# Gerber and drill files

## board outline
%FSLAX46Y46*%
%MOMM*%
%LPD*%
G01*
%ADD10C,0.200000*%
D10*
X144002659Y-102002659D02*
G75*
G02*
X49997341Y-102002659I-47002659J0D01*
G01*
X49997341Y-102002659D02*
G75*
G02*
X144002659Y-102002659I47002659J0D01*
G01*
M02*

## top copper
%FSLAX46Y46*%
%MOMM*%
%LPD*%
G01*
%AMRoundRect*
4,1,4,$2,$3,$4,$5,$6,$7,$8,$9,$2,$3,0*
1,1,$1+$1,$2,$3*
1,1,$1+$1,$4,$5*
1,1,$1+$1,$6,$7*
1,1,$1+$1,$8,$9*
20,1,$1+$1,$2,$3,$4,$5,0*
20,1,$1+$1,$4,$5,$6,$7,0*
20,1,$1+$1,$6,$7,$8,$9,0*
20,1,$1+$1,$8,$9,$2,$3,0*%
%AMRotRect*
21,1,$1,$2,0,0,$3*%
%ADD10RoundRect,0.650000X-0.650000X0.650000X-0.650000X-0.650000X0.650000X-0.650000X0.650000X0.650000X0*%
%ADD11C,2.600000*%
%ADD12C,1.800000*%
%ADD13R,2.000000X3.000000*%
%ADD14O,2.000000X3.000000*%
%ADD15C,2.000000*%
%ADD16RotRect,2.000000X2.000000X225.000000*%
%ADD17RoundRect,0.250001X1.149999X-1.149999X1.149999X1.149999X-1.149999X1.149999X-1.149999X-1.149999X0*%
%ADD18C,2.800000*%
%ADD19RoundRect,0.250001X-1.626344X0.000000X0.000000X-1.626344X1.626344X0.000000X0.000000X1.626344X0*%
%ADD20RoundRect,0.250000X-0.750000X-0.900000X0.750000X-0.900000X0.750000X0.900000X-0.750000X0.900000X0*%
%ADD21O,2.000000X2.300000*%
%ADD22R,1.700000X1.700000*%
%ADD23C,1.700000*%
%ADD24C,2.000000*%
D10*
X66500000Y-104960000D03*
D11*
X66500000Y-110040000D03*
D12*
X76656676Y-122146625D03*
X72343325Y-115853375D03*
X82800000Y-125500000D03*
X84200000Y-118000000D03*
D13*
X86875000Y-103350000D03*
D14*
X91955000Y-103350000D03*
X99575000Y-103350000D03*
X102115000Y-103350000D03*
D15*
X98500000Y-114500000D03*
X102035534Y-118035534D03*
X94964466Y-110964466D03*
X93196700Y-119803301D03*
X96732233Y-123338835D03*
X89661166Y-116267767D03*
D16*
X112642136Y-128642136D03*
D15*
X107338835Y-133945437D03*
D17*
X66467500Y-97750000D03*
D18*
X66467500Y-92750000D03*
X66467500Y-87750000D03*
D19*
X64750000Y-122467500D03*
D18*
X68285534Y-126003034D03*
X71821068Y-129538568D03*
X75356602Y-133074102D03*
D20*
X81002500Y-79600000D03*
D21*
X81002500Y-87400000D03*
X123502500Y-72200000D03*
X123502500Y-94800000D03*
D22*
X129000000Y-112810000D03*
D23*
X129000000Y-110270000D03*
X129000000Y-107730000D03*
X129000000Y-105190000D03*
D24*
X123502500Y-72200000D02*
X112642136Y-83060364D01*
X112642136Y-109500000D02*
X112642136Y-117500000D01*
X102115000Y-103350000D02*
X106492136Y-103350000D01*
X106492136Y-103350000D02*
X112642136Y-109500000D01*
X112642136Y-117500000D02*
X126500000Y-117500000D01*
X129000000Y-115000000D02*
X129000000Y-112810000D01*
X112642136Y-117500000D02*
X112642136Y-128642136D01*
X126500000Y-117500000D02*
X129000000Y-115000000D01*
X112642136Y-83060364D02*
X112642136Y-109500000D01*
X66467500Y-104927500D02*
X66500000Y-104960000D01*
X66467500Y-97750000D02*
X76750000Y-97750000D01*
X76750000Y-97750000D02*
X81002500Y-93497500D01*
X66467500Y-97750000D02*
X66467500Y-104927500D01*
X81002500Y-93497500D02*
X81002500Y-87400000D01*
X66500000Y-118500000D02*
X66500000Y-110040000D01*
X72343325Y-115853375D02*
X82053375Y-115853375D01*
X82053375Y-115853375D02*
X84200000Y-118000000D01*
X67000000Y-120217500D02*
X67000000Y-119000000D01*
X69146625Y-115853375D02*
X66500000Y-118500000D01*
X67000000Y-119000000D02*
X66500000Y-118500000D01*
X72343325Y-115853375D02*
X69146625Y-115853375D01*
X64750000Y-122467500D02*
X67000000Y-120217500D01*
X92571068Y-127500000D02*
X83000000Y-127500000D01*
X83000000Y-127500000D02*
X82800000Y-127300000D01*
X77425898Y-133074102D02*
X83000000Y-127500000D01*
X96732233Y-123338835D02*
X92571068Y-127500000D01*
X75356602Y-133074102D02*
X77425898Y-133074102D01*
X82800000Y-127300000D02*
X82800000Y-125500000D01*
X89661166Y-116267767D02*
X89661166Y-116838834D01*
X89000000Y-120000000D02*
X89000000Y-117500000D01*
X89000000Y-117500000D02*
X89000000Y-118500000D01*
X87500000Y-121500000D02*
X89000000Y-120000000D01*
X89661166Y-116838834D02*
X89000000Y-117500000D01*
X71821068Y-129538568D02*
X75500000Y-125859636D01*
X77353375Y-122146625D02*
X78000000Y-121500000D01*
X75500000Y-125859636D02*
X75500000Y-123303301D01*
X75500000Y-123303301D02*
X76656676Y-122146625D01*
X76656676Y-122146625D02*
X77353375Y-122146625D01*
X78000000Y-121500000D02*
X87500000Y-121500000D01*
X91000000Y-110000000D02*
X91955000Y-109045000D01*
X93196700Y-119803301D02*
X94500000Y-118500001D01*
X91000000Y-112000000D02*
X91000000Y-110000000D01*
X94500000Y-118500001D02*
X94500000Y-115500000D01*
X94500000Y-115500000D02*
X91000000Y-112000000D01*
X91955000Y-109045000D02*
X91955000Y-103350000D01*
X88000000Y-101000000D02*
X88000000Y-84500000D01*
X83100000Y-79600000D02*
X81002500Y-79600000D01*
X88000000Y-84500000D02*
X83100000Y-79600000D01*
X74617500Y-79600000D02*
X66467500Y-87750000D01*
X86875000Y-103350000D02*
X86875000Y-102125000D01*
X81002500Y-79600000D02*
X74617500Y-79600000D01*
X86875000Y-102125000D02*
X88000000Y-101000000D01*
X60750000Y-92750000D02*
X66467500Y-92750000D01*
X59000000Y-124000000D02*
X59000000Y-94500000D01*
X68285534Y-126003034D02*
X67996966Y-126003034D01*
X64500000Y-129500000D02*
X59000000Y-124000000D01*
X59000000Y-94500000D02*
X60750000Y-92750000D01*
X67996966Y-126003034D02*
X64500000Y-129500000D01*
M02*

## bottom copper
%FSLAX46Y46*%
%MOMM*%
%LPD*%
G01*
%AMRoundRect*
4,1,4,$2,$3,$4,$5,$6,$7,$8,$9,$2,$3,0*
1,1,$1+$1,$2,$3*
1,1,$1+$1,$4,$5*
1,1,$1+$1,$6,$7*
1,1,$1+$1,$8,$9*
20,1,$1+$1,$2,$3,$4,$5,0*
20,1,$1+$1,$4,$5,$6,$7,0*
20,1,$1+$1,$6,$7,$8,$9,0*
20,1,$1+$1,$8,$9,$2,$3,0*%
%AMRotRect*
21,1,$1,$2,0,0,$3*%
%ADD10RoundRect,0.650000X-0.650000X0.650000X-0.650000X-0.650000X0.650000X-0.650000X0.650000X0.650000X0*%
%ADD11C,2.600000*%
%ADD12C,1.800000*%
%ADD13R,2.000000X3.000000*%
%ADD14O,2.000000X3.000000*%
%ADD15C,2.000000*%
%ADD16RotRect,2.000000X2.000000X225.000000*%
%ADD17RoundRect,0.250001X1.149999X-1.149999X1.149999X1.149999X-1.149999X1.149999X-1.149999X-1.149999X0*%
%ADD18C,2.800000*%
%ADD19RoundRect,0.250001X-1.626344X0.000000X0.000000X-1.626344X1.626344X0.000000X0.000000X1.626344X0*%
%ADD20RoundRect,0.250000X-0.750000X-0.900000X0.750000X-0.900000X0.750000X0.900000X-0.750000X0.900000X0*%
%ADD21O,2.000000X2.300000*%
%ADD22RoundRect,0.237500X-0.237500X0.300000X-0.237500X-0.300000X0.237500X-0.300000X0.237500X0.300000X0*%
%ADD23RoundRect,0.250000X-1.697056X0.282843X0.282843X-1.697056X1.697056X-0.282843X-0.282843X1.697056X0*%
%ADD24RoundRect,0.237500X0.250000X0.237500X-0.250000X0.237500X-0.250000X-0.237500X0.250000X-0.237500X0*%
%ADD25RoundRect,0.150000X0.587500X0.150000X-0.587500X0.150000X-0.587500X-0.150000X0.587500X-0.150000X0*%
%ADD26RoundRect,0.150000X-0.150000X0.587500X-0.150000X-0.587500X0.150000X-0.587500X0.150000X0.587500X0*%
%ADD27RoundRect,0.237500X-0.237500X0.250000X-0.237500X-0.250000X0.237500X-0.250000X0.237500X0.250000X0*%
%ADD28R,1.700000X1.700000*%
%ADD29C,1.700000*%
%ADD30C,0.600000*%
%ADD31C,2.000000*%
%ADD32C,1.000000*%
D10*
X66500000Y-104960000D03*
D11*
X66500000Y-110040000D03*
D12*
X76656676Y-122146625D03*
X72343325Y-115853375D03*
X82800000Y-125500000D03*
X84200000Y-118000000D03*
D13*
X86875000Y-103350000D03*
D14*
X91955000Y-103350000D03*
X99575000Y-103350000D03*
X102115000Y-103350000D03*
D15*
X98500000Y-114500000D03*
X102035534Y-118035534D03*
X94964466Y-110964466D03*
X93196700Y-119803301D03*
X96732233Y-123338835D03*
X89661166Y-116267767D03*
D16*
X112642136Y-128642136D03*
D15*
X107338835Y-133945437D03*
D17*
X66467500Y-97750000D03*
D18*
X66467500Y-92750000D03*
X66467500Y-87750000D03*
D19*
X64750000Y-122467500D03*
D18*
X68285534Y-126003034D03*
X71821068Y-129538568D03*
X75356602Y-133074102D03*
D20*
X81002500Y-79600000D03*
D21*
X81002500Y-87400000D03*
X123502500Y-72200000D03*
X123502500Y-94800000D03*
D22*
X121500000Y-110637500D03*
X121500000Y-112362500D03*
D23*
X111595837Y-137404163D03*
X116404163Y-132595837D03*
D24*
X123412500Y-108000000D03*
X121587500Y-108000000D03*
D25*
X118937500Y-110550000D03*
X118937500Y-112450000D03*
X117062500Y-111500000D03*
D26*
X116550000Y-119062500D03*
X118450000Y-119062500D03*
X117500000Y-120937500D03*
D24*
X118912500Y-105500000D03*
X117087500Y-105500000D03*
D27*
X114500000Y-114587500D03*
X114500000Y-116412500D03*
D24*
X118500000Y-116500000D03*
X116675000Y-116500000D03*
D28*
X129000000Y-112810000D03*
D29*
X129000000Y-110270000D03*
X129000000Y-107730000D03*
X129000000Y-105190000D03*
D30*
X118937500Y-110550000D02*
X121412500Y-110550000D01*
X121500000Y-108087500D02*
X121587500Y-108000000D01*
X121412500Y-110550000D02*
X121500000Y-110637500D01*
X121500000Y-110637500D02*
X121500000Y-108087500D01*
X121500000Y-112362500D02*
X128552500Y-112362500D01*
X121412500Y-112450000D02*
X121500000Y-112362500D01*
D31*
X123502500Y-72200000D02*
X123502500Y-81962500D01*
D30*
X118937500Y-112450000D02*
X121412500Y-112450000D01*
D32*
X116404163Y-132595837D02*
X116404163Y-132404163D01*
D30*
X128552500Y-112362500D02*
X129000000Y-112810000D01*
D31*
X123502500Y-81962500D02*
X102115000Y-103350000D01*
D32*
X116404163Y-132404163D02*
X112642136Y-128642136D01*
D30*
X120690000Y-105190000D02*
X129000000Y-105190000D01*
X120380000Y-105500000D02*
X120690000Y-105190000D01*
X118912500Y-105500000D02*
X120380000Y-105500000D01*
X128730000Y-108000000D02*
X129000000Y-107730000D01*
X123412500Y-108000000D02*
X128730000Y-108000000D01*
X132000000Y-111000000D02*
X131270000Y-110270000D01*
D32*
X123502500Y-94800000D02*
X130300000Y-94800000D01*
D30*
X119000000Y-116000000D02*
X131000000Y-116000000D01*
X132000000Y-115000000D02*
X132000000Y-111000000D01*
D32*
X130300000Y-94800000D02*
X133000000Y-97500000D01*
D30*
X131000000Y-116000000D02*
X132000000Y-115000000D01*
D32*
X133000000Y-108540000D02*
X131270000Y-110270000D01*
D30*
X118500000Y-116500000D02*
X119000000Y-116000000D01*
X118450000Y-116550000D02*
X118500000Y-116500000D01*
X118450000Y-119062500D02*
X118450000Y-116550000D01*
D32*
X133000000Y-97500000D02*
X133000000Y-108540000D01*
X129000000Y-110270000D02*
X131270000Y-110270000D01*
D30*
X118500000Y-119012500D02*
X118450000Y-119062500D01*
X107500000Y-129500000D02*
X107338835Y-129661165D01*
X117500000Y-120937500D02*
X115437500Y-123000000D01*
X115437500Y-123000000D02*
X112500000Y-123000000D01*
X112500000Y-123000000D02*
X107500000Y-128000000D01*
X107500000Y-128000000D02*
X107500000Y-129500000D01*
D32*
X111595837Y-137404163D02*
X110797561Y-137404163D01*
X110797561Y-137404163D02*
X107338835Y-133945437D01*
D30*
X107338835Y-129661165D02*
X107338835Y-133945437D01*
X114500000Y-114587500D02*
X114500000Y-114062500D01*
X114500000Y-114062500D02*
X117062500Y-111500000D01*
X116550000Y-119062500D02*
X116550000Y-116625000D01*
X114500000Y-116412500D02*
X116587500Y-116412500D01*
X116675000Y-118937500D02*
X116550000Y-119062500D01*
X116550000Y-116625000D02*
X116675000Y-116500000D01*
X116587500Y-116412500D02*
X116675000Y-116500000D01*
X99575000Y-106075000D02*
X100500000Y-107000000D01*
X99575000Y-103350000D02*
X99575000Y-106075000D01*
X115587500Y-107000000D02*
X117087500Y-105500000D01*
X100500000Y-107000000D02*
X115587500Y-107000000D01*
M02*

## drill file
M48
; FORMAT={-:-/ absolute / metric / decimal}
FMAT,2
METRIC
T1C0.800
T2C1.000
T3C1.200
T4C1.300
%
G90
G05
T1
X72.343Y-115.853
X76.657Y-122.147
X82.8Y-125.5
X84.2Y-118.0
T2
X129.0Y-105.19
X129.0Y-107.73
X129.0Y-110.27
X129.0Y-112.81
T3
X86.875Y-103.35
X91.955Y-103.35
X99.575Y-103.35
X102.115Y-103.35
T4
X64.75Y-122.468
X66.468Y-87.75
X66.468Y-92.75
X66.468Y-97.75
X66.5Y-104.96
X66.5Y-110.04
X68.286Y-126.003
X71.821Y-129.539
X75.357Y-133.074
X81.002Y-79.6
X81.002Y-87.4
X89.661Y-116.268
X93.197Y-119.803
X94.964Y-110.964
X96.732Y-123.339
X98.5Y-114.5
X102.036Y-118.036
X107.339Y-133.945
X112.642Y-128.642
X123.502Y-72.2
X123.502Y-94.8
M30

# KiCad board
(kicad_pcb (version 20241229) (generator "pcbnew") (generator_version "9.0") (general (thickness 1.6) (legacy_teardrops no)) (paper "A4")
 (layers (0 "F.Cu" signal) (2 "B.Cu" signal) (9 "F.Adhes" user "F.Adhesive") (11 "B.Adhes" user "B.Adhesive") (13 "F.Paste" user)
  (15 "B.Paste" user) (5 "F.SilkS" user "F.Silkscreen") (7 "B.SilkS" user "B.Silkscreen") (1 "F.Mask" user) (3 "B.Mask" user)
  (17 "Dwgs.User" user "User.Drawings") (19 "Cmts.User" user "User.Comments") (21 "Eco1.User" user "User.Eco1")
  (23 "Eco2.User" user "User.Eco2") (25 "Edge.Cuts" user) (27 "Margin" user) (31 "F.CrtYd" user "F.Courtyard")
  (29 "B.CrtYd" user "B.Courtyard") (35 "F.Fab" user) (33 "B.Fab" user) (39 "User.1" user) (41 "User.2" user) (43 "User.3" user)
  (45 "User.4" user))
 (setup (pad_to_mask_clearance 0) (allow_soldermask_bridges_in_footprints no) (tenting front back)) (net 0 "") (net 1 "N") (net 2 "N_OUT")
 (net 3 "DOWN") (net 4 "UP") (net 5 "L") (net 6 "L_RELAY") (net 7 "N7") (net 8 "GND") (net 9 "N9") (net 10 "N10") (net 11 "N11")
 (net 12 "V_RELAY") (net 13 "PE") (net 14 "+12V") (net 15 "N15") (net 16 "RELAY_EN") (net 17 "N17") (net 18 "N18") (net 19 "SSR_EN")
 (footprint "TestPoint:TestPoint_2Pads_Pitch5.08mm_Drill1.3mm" (layer "F.Cu") (at 66.5 104.96 -90)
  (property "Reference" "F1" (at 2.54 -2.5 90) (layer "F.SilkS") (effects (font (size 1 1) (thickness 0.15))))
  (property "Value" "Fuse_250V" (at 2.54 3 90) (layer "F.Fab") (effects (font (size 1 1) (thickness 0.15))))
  (pad "1" thru_hole roundrect (at 0 0 270) (size 2.6 2.6) (drill 1.3) (layers "*.Cu" "*.Mask") (remove_unused_layers no)
   (roundrect_rratio 0.25) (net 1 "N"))
  (pad "2" thru_hole circle (at 5.08 0 270) (size 2.6 2.6) (drill 1.3) (layers "*.Cu" "*.Mask") (remove_unused_layers no) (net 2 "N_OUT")))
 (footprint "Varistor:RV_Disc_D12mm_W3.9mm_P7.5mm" (layer "F.Cu") (at 76.656676 122.146625 135)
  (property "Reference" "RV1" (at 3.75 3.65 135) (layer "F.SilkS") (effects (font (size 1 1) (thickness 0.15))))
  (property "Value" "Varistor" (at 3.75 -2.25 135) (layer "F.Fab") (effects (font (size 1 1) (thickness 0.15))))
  (pad "1" thru_hole circle (at 0 0 135) (size 1.8 1.8) (drill 0.8) (layers "*.Cu" "*.Mask") (remove_unused_layers no) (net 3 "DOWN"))
  (pad "2" thru_hole circle (at 7.499999 1.4 135) (size 1.8 1.8) (drill 0.8) (layers "*.Cu" "*.Mask") (remove_unused_layers no)
   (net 2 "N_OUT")))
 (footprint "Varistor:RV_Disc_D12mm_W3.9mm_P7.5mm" (layer "F.Cu") (at 82.8 125.5 90)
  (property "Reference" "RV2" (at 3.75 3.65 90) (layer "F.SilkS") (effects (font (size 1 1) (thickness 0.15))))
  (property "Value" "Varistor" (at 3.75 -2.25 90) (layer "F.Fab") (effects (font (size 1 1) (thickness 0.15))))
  (pad "1" thru_hole circle (at 0 0 90) (size 1.8 1.8) (drill 0.8) (layers "*.Cu" "*.Mask") (remove_unused_layers no) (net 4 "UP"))
  (pad "2" thru_hole circle (at 7.5 1.4 90) (size 1.8 1.8) (drill 0.8) (layers "*.Cu" "*.Mask") (remove_unused_layers no) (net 2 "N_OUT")))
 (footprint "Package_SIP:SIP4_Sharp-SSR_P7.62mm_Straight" (layer "F.Cu") (at 86.875 103.35)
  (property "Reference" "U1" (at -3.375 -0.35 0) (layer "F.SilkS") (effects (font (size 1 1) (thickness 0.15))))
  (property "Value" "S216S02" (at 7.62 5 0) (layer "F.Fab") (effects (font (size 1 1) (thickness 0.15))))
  (pad "1" thru_hole rect (at 0 0) (size 2 3) (drill 1.2) (layers "*.Cu" "*.Mask") (remove_unused_layers no) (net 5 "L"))
  (pad "2" thru_hole oval (at 5.08 0) (size 2 3) (drill 1.2) (layers "*.Cu" "*.Mask") (remove_unused_layers no) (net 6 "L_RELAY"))
  (pad "3" thru_hole oval (at 12.7 0) (size 2 3) (drill 1.2) (layers "*.Cu" "*.Mask") (remove_unused_layers no) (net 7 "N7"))
  (pad "4" thru_hole oval (at 15.24 0) (size 2 3) (drill 1.2) (layers "*.Cu" "*.Mask") (remove_unused_layers no) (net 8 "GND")))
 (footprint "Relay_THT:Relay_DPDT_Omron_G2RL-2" (layer "F.Cu") (at 112.642136 128.642136 -135)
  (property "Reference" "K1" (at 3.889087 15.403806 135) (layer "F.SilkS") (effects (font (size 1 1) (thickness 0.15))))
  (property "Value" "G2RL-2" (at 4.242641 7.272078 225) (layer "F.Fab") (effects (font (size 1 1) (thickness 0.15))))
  (pad "11" thru_hole circle (at 0 20.000001 225) (size 2 2) (drill 1.3) (layers "*.Cu" "*.Mask") (remove_unused_layers no) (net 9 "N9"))
  (pad "12" thru_hole circle (at 0 15 225) (size 2 2) (drill 1.3) (layers "*.Cu" "*.Mask") (remove_unused_layers no) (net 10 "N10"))
  (pad "14" thru_hole circle (at 0 25.000001 225) (size 2 2) (drill 1.3) (layers "*.Cu" "*.Mask") (remove_unused_layers no) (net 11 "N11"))
  (pad "21" thru_hole circle (at 7.499999 20 225) (size 2 2) (drill 1.3) (layers "*.Cu" "*.Mask") (remove_unused_layers no)
   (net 6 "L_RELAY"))
  (pad "22" thru_hole circle (at 7.5 15 225) (size 2 2) (drill 1.3) (layers "*.Cu" "*.Mask") (remove_unused_layers no) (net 4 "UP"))
  (pad "24" thru_hole circle (at 7.499999 25 225) (size 2 2) (drill 1.3) (layers "*.Cu" "*.Mask") (remove_unused_layers no) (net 3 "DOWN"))
  (pad "A1" thru_hole rect (at 0 0 225) (size 2 2) (drill 1.3) (layers "*.Cu" "*.Mask") (remove_unused_layers no) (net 8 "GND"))
  (pad "A2" thru_hole circle (at 7.5 0 225) (size 2 2) (drill 1.3) (layers "*.Cu" "*.Mask") (remove_unused_layers no) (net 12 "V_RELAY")))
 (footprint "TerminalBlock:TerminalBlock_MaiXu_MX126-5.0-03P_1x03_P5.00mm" (layer "F.Cu") (at 66.4675 97.75 90)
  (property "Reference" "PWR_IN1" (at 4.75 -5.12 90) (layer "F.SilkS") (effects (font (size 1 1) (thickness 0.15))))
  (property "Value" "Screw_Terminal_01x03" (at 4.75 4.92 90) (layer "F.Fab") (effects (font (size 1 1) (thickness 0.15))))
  (pad "1" thru_hole roundrect (at 0 0 90) (size 2.8 2.8) (drill 1.3) (layers "*.Cu" "*.Mask") (remove_unused_layers no)
   (roundrect_rratio 0.089286) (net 1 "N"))
  (pad "2" thru_hole circle (at 5 0 90) (size 2.8 2.8) (drill 1.3) (layers "*.Cu" "*.Mask") (remove_unused_layers no) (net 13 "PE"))
  (pad "3" thru_hole circle (at 10 0 90) (size 2.8 2.8) (drill 1.3) (layers "*.Cu" "*.Mask") (remove_unused_layers no) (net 5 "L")))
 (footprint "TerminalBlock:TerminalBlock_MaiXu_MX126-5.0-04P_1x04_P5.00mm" (layer "F.Cu") (at 64.75 122.4675 -45)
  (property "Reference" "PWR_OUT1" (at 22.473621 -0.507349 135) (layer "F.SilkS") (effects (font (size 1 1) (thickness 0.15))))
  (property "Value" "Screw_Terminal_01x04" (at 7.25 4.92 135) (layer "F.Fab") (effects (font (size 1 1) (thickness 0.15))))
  (pad "1" thru_hole roundrect (at 0 0 315) (size 2.8 2.8) (drill 1.3) (layers "*.Cu" "*.Mask") (remove_unused_layers no)
   (roundrect_rratio 0.089286) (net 2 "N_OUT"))
  (pad "2" thru_hole circle (at 5 0 315) (size 2.8 2.8) (drill 1.3) (layers "*.Cu" "*.Mask") (remove_unused_layers no) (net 13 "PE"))
  (pad "3" thru_hole circle (at 10 0 315) (size 2.8 2.8) (drill 1.3) (layers "*.Cu" "*.Mask") (remove_unused_layers no) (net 3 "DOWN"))
  (pad "4" thru_hole circle (at 15 0 315) (size 2.8 2.8) (drill 1.3) (layers "*.Cu" "*.Mask") (remove_unused_layers no) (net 4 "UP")))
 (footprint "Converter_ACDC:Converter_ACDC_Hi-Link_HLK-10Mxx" (layer "F.Cu") (at 81.0025 79.6)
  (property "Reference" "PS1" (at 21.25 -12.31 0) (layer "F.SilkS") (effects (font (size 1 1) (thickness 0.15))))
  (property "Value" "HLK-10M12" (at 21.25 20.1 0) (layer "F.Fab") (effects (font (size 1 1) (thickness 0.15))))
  (pad "1" thru_hole roundrect (at 0 0) (size 2 2.3) (drill 1.3) (layers "*.Cu" "*.Mask") (remove_unused_layers no) (roundrect_rratio 0.125)
   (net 5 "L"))
  (pad "2" thru_hole oval (at 0 7.8) (size 2 2.3) (drill 1.3) (layers "*.Cu" "*.Mask") (remove_unused_layers no) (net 1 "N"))
  (pad "3" thru_hole oval (at 42.5 -7.4) (size 2 2.3) (drill 1.3) (layers "*.Cu" "*.Mask") (remove_unused_layers no) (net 8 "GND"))
  (pad "4" thru_hole oval (at 42.5 15.2) (size 2 2.3) (drill 1.3) (layers "*.Cu" "*.Mask") (remove_unused_layers no) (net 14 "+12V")))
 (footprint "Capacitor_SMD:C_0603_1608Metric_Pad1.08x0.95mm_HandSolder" (layer "B.Cu") (at 121.5 111.5 -90)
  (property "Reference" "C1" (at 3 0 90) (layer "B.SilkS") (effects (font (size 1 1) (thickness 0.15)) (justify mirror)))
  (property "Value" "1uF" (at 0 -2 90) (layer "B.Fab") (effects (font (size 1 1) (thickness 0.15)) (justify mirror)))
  (pad "1" smd roundrect (at -0.8625 0 270) (size 1.075 0.95) (layers "B.Cu" "B.Mask" "B.Paste") (roundrect_rratio 0.25) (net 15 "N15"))
  (pad "2" smd roundrect (at 0.8625 0 270) (size 1.075 0.95) (layers "B.Cu" "B.Mask" "B.Paste") (roundrect_rratio 0.25) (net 8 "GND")))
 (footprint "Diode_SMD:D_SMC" (layer "B.Cu") (at 114 135 45)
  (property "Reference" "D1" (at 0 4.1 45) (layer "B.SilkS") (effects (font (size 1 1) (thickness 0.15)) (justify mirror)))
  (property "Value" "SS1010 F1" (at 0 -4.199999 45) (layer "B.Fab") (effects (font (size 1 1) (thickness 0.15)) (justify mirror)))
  (pad "1" smd roundrect (at -3.4 0 315) (size 3.3 2.5) (layers "B.Cu" "B.Mask" "B.Paste") (roundrect_rratio 0.1) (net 12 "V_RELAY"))
  (pad "2" smd roundrect (at 3.4 0 315) (size 3.3 2.5) (layers "B.Cu" "B.Mask" "B.Paste") (roundrect_rratio 0.1) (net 8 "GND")))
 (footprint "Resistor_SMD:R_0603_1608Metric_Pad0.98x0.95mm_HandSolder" (layer "B.Cu") (at 122.5 108 180)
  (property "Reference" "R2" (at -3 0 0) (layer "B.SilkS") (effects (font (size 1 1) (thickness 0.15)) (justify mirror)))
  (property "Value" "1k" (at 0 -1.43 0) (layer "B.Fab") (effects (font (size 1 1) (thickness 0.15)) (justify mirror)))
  (pad "1" smd roundrect (at -0.9125 0 180) (size 0.975 0.95) (layers "B.Cu" "B.Mask" "B.Paste") (roundrect_rratio 0.25) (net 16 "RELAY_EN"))
  (pad "2" smd roundrect (at 0.9125 0 180) (size 0.975 0.95) (layers "B.Cu" "B.Mask" "B.Paste") (roundrect_rratio 0.25) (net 15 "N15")))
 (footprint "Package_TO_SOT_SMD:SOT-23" (layer "B.Cu") (at 118 111.5 180)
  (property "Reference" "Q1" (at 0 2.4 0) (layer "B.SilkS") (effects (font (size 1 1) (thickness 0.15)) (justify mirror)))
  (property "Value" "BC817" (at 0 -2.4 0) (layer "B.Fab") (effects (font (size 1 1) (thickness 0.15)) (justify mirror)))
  (pad "1" smd roundrect (at -0.9375 0.95 180) (size 1.475 0.6) (layers "B.Cu" "B.Mask" "B.Paste") (roundrect_rratio 0.25) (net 15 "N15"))
  (pad "2" smd roundrect (at -0.9375 -0.95 180) (size 1.475 0.6) (layers "B.Cu" "B.Mask" "B.Paste") (roundrect_rratio 0.25) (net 8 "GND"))
  (pad "3" smd roundrect (at 0.9375 0 180) (size 1.475 0.6) (layers "B.Cu" "B.Mask" "B.Paste") (roundrect_rratio 0.25) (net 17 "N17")))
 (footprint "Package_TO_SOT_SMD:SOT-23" (layer "B.Cu") (at 117.5 120 -90)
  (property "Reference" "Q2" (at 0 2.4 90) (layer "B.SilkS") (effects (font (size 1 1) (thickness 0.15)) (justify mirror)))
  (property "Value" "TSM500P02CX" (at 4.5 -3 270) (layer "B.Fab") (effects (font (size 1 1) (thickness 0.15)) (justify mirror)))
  (pad "1" smd roundrect (at -0.9375 0.95 270) (size 1.475 0.6) (layers "B.Cu" "B.Mask" "B.Paste") (roundrect_rratio 0.25) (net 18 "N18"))
  (pad "2" smd roundrect (at -0.9375 -0.95 270) (size 1.475 0.6) (layers "B.Cu" "B.Mask" "B.Paste") (roundrect_rratio 0.25) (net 14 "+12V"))
  (pad "3" smd roundrect (at 0.9375 0 270) (size 1.475 0.6) (layers "B.Cu" "B.Mask" "B.Paste") (roundrect_rratio 0.25) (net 12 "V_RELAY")))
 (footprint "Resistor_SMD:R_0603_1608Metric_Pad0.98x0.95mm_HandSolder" (layer "B.Cu") (at 118 105.5 180)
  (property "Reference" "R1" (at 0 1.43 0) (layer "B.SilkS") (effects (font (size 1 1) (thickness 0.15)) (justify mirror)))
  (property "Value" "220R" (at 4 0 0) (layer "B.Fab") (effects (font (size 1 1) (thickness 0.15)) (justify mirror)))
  (pad "1" smd roundrect (at -0.9125 0 180) (size 0.975 0.95) (layers "B.Cu" "B.Mask" "B.Paste") (roundrect_rratio 0.25) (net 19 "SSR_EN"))
  (pad "2" smd roundrect (at 0.9125 0 180) (size 0.975 0.95) (layers "B.Cu" "B.Mask" "B.Paste") (roundrect_rratio 0.25) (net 7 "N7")))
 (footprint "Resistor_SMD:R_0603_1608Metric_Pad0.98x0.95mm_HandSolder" (layer "B.Cu") (at 114.5 115.5 -90)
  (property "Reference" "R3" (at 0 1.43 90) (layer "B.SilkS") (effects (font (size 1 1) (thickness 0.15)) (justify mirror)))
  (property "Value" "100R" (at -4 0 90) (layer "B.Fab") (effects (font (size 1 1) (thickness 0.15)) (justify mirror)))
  (pad "1" smd roundrect (at -0.9125 0 270) (size 0.975 0.95) (layers "B.Cu" "B.Mask" "B.Paste") (roundrect_rratio 0.25) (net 17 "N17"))
  (pad "2" smd roundrect (at 0.9125 0 270) (size 0.975 0.95) (layers "B.Cu" "B.Mask" "B.Paste") (roundrect_rratio 0.25) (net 18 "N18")))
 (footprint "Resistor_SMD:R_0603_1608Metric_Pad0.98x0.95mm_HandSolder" (layer "B.Cu") (at 117.5875 116.5 180)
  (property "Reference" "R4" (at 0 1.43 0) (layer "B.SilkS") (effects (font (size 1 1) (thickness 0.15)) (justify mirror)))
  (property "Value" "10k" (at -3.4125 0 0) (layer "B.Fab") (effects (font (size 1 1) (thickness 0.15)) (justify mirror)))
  (pad "1" smd roundrect (at -0.9125 0 180) (size 0.975 0.95) (layers "B.Cu" "B.Mask" "B.Paste") (roundrect_rratio 0.25) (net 14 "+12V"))
  (pad "2" smd roundrect (at 0.9125 0 180) (size 0.975 0.95) (layers "B.Cu" "B.Mask" "B.Paste") (roundrect_rratio 0.25) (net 18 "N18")))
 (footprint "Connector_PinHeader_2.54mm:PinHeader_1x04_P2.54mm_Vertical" (layer "B.Cu") (at 129 112.81)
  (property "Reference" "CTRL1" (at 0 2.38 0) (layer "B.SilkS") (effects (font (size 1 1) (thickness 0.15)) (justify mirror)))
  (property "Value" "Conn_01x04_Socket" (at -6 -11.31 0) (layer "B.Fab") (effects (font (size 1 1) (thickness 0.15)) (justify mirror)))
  (pad "1" thru_hole rect (at 0 0) (size 1.7 1.7) (drill 1) (layers "*.Cu" "*.Mask") (remove_unused_layers no) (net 8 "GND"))
  (pad "2" thru_hole circle (at 0 -2.54) (size 1.7 1.7) (drill 1) (layers "*.Cu" "*.Mask") (remove_unused_layers no) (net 14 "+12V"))
  (pad "3" thru_hole circle (at 0 -5.08) (size 1.7 1.7) (drill 1) (layers "*.Cu" "*.Mask") (remove_unused_layers no) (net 16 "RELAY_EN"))
  (pad "4" thru_hole circle (at 0 -7.62) (size 1.7 1.7) (drill 1) (layers "*.Cu" "*.Mask") (remove_unused_layers no) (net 19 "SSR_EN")))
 (gr_circle (center 97 102.002659) (end 144 102.502659) (stroke (width 0.2) (type solid)) (fill no) (layer "Edge.Cuts"))
 (segment (start 118.9375 110.55) (end 121.4125 110.55) (width 0.6) (layer "B.Cu") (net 15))
 (segment (start 121.5 108.0875) (end 121.5875 108) (width 0.6) (layer "B.Cu") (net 15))
 (segment (start 121.4125 110.55) (end 121.5 110.6375) (width 0.6) (layer "B.Cu") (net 15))
 (segment (start 121.5 110.6375) (end 121.5 108.0875) (width 0.6) (layer "B.Cu") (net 15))
 (segment (start 123.5025 72.2) (end 112.642136 83.060364) (width 2) (layer "F.Cu") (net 8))
 (segment (start 112.642136 109.5) (end 112.642136 117.5) (width 2) (layer "F.Cu") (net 8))
 (segment (start 102.115 103.35) (end 106.492136 103.35) (width 2) (layer "F.Cu") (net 8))
 (segment (start 106.492136 103.35) (end 112.642136 109.5) (width 2) (layer "F.Cu") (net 8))
 (segment (start 112.642136 117.5) (end 126.5 117.5) (width 2) (layer "F.Cu") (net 8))
 (segment (start 129 115) (end 129 112.81) (width 2) (layer "F.Cu") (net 8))
 (segment (start 112.642136 117.5) (end 112.642136 128.642136) (width 2) (layer "F.Cu") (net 8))
 (segment (start 126.5 117.5) (end 129 115) (width 2) (layer "F.Cu") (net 8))
 (segment (start 112.642136 83.060364) (end 112.642136 109.5) (width 2) (layer "F.Cu") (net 8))
 (segment (start 121.5 112.3625) (end 128.5525 112.3625) (width 0.6) (layer "B.Cu") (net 8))
 (segment (start 121.4125 112.45) (end 121.5 112.3625) (width 0.6) (layer "B.Cu") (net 8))
 (segment (start 123.5025 72.2) (end 123.5025 81.9625) (width 2) (layer "B.Cu") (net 8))
 (segment (start 118.9375 112.45) (end 121.4125 112.45) (width 0.6) (layer "B.Cu") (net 8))
 (segment (start 116.404163 132.595837) (end 116.404163 132.404163) (width 1) (layer "B.Cu") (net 8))
 (segment (start 128.5525 112.3625) (end 129 112.81) (width 0.6) (layer "B.Cu") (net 8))
 (segment (start 123.5025 81.9625) (end 102.115 103.35) (width 2) (layer "B.Cu") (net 8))
 (segment (start 116.404163 132.404163) (end 112.642136 128.642136) (width 1) (layer "B.Cu") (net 8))
 (segment (start 120.69 105.19) (end 129 105.19) (width 0.6) (layer "B.Cu") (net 19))
 (segment (start 120.38 105.5) (end 120.69 105.19) (width 0.6) (layer "B.Cu") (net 19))
 (segment (start 118.9125 105.5) (end 120.38 105.5) (width 0.6) (layer "B.Cu") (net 19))
 (segment (start 128.73 108) (end 129 107.73) (width 0.6) (layer "B.Cu") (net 16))
 (segment (start 123.4125 108) (end 128.73 108) (width 0.6) (layer "B.Cu") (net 16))
 (segment (start 132 111) (end 131.27 110.27) (width 0.6) (layer "B.Cu") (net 14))
 (segment (start 123.5025 94.8) (end 130.3 94.8) (width 1) (layer "B.Cu") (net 14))
 (segment (start 119 116) (end 131 116) (width 0.6) (layer "B.Cu") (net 14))
 (segment (start 132 115) (end 132 111) (width 0.6) (layer "B.Cu") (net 14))
 (segment (start 130.3 94.8) (end 133 97.5) (width 1) (layer "B.Cu") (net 14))
 (segment (start 131 116) (end 132 115) (width 0.6) (layer "B.Cu") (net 14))
 (segment (start 133 108.54) (end 131.27 110.27) (width 1) (layer "B.Cu") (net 14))
 (segment (start 118.5 116.5) (end 119 116) (width 0.6) (layer "B.Cu") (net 14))
 (segment (start 118.45 116.55) (end 118.5 116.5) (width 0.6) (layer "B.Cu") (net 14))
 (segment (start 118.45 119.0625) (end 118.45 116.55) (width 0.6) (layer "B.Cu") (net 14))
 (segment (start 133 97.5) (end 133 108.54) (width 1) (layer "B.Cu") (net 14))
 (segment (start 129 110.27) (end 131.27 110.27) (width 1) (layer "B.Cu") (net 14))
 (segment (start 118.5 119.0125) (end 118.45 119.0625) (width 0.6) (layer "B.Cu") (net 14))
 (segment (start 107.5 129.5) (end 107.338835 129.661165) (width 0.6) (layer "B.Cu") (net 12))
 (segment (start 117.5 120.9375) (end 115.4375 123) (width 0.6) (layer "B.Cu") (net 12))
 (segment (start 115.4375 123) (end 112.5 123) (width 0.6) (layer "B.Cu") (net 12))
 (segment (start 112.5 123) (end 107.5 128) (width 0.6) (layer "B.Cu") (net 12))
 (segment (start 107.5 128) (end 107.5 129.5) (width 0.6) (layer "B.Cu") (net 12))
 (segment (start 111.595837 137.404163) (end 110.797561 137.404163) (width 1) (layer "B.Cu") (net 12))
 (segment (start 110.797561 137.404163) (end 107.338835 133.945437) (width 1) (layer "B.Cu") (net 12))
 (segment (start 107.338835 129.661165) (end 107.338835 133.945437) (width 0.6) (layer "B.Cu") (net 12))
 (segment (start 66.4675 104.9275) (end 66.5 104.96) (width 2) (layer "F.Cu") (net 1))
 (segment (start 66.4675 97.75) (end 76.75 97.75) (width 2) (layer "F.Cu") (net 1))
 (segment (start 76.75 97.75) (end 81.0025 93.4975) (width 2) (layer "F.Cu") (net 1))
 (segment (start 66.4675 97.75) (end 66.4675 104.9275) (width 2) (layer "F.Cu") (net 1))
 (segment (start 81.0025 93.4975) (end 81.0025 87.4) (width 2) (layer "F.Cu") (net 1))
 (segment (start 66.5 118.5) (end 66.5 110.04) (width 2) (layer "F.Cu") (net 2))
 (segment (start 72.343325 115.853375) (end 82.053375 115.853375) (width 2) (layer "F.Cu") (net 2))
 (segment (start 82.053375 115.853375) (end 84.2 118) (width 2) (layer "F.Cu") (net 2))
 (segment (start 67 120.2175) (end 67 119) (width 2) (layer "F.Cu") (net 2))
 (segment (start 69.146625 115.853375) (end 66.5 118.5) (width 2) (layer "F.Cu") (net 2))
 (segment (start 67 119) (end 66.5 118.5) (width 2) (layer "F.Cu") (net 2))
 (segment (start 72.343325 115.853375) (end 69.146625 115.853375) (width 2) (layer "F.Cu") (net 2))
 (segment (start 64.75 122.4675) (end 67 120.2175) (width 2) (layer "F.Cu") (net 2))
 (segment (start 92.571068 127.5) (end 83 127.5) (width 2) (layer "F.Cu") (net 4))
 (segment (start 83 127.5) (end 82.8 127.3) (width 2) (layer "F.Cu") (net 4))
 (segment (start 77.425898 133.074102) (end 83 127.5) (width 2) (layer "F.Cu") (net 4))
 (segment (start 96.732233 123.338835) (end 92.571068 127.5) (width 2) (layer "F.Cu") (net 4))
 (segment (start 75.356602 133.074102) (end 77.425898 133.074102) (width 2) (layer "F.Cu") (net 4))
 (segment (start 82.8 127.3) (end 82.8 125.5) (width 2) (layer "F.Cu") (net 4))
 (segment (start 89.661166 116.267767) (end 89.661166 116.838834) (width 2) (layer "F.Cu") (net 3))
 (segment (start 89 120) (end 89 117.5) (width 2) (layer "F.Cu") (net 3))
 (segment (start 89 117.5) (end 89 118.5) (width 2) (layer "F.Cu") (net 3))
 (segment (start 87.5 121.5) (end 89 120) (width 2) (layer "F.Cu") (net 3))
 (segment (start 89.661166 116.838834) (end 89 117.5) (width 2) (layer "F.Cu") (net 3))
 (segment (start 71.821068 129.538568) (end 75.5 125.859636) (width 2) (layer "F.Cu") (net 3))
 (segment (start 77.353375 122.146625) (end 78 121.5) (width 2) (layer "F.Cu") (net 3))
 (segment (start 75.5 125.859636) (end 75.5 123.303301) (width 2) (layer "F.Cu") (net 3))
 (segment (start 75.5 123.303301) (end 76.656676 122.146625) (width 2) (layer "F.Cu") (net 3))
 (segment (start 76.656676 122.146625) (end 77.353375 122.146625) (width 2) (layer "F.Cu") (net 3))
 (segment (start 78 121.5) (end 87.5 121.5) (width 2) (layer "F.Cu") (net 3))
 (segment (start 91 110) (end 91.955 109.045) (width 2) (layer "F.Cu") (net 6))
 (segment (start 93.1967 119.803301) (end 94.5 118.500001) (width 2) (layer "F.Cu") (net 6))
 (segment (start 91 112) (end 91 110) (width 2) (layer "F.Cu") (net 6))
 (segment (start 94.5 118.500001) (end 94.5 115.5) (width 2) (layer "F.Cu") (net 6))
 (segment (start 94.5 115.5) (end 91 112) (width 2) (layer "F.Cu") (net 6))
 (segment (start 91.955 109.045) (end 91.955 103.35) (width 2) (layer "F.Cu") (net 6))
 (segment (start 88 101) (end 88 84.5) (width 2) (layer "F.Cu") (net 5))
 (segment (start 83.1 79.6) (end 81.0025 79.6) (width 2) (layer "F.Cu") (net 5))
 (segment (start 88 84.5) (end 83.1 79.6) (width 2) (layer "F.Cu") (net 5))
 (segment (start 74.6175 79.6) (end 66.4675 87.75) (width 2) (layer "F.Cu") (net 5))
 (segment (start 86.875 103.35) (end 86.875 102.125) (width 2) (layer "F.Cu") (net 5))
 (segment (start 81.0025 79.6) (end 74.6175 79.6) (width 2) (layer "F.Cu") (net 5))
 (segment (start 86.875 102.125) (end 88 101) (width 2) (layer "F.Cu") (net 5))
 (segment (start 60.75 92.75) (end 66.4675 92.75) (width 2) (layer "F.Cu") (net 13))
 (segment (start 59 124) (end 59 94.5) (width 2) (layer "F.Cu") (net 13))
 (segment (start 68.285534 126.003034) (end 67.996966 126.003034) (width 2) (layer "F.Cu") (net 13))
 (segment (start 64.5 129.5) (end 59 124) (width 2) (layer "F.Cu") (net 13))
 (segment (start 59 94.5) (end 60.75 92.75) (width 2) (layer "F.Cu") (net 13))
 (segment (start 67.996966 126.003034) (end 64.5 129.5) (width 2) (layer "F.Cu") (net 13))
 (segment (start 114.5 114.5875) (end 114.5 114.0625) (width 0.6) (layer "B.Cu") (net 17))
 (segment (start 114.5 114.0625) (end 117.0625 111.5) (width 0.6) (layer "B.Cu") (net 17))
 (segment (start 116.55 119.0625) (end 116.55 116.625) (width 0.6) (layer "B.Cu") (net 18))
 (segment (start 114.5 116.4125) (end 116.5875 116.4125) (width 0.6) (layer "B.Cu") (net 18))
 (segment (start 116.675 118.9375) (end 116.55 119.0625) (width 0.6) (layer "B.Cu") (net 18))
 (segment (start 116.55 116.625) (end 116.675 116.5) (width 0.6) (layer "B.Cu") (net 18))
 (segment (start 116.5875 116.4125) (end 116.675 116.5) (width 0.6) (layer "B.Cu") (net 18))
 (segment (start 99.575 106.075) (end 100.5 107) (width 0.6) (layer "B.Cu") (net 7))
 (segment (start 99.575 103.35) (end 99.575 106.075) (width 0.6) (layer "B.Cu") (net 7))
 (segment (start 115.5875 107) (end 117.0875 105.5) (width 0.6) (layer "B.Cu") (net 7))
 (segment (start 100.5 107) (end 115.5875 107) (width 0.6) (layer "B.Cu") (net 7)))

